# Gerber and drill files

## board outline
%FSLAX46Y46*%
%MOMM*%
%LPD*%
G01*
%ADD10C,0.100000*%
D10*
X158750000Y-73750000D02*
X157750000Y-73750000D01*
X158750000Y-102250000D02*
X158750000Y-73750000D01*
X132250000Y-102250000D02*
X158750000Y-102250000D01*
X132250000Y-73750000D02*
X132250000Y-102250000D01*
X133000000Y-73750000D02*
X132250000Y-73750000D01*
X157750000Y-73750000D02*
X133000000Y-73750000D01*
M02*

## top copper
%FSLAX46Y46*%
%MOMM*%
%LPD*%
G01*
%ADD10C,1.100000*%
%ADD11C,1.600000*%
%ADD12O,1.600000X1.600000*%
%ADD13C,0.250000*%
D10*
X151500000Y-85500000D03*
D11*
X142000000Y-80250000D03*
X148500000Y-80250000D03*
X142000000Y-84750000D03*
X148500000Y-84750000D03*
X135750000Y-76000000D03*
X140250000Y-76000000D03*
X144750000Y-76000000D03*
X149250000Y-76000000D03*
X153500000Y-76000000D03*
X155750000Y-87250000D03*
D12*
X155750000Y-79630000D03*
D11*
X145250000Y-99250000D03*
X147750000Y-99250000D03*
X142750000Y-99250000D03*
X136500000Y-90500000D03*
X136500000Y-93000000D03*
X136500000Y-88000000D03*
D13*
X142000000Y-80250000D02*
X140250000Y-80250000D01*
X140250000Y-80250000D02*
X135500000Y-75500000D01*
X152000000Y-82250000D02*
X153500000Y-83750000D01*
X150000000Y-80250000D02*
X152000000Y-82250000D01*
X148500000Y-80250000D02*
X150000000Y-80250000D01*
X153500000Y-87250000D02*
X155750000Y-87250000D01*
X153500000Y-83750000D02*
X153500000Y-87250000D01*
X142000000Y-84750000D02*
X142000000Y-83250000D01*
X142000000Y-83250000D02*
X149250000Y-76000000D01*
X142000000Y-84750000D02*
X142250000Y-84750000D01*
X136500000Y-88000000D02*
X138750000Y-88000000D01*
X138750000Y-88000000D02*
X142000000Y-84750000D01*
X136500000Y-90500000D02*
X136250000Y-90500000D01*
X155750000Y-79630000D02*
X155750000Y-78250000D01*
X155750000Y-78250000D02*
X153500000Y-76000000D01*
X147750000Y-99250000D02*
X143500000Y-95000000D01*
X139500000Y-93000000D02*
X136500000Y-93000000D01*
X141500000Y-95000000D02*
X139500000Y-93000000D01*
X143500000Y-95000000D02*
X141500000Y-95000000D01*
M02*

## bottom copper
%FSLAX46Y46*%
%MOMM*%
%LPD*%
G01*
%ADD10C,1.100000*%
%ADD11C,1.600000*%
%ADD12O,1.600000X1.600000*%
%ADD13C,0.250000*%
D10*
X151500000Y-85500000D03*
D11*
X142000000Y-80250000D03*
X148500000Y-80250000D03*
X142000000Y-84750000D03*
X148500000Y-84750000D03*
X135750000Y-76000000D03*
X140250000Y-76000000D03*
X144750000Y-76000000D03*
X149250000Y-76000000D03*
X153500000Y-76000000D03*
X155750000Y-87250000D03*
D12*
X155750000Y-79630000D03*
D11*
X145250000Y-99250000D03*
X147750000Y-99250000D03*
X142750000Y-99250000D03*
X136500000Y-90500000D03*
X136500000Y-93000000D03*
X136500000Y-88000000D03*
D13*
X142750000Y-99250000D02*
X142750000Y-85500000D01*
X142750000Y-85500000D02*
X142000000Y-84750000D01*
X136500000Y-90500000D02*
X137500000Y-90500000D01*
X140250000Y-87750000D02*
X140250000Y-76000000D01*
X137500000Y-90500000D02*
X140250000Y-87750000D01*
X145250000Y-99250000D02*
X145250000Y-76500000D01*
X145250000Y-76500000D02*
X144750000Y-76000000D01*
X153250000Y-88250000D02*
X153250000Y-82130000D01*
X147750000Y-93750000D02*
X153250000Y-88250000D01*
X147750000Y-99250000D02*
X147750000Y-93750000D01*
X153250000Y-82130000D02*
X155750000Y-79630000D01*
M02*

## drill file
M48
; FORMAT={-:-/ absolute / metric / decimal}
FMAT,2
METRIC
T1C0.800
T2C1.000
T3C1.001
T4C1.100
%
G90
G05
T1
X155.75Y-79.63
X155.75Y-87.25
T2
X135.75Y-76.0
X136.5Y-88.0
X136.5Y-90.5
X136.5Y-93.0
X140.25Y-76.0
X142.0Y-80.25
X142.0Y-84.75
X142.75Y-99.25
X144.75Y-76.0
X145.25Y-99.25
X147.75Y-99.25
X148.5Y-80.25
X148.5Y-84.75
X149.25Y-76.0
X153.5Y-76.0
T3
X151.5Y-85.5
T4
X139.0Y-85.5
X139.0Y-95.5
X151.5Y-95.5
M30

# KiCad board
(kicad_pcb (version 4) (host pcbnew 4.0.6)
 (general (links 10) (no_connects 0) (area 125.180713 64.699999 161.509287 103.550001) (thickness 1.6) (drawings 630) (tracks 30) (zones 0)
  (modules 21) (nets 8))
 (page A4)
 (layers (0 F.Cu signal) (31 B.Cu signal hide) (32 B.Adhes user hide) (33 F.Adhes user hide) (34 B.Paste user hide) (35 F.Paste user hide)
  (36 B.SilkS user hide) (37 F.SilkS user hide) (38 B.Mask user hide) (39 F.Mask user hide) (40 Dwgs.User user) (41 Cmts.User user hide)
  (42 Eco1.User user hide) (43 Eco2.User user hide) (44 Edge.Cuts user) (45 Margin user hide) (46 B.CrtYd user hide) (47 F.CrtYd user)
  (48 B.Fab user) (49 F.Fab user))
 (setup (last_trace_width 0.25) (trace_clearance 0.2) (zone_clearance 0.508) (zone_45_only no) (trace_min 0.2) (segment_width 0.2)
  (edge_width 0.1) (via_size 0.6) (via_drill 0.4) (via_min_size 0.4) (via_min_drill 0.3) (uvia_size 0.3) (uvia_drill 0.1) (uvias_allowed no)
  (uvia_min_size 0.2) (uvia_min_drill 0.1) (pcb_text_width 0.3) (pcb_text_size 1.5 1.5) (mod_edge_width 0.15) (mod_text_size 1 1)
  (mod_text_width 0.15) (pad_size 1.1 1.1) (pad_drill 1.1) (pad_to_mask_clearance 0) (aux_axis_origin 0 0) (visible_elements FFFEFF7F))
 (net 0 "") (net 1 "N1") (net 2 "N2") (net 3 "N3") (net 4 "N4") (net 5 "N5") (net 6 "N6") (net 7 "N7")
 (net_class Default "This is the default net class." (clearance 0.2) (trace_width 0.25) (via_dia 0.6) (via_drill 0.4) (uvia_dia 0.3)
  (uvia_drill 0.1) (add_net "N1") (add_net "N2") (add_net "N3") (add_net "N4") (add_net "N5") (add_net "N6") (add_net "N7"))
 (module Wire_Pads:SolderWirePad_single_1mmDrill (layer F.Cu) (at 151.5 95.5)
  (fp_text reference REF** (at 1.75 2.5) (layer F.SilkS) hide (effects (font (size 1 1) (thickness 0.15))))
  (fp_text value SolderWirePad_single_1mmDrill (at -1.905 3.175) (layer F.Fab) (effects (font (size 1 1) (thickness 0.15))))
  (pad "" np_thru_hole circle (at 0 0) (size 1.1 1.1) (drill 1.1) (layers *.Cu *.Mask)))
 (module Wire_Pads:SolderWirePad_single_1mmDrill (layer F.Cu) (at 139 95.5)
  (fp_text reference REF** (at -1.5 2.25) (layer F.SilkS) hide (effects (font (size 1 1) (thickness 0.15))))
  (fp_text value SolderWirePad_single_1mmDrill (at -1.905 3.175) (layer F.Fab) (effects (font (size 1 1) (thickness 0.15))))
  (pad "" np_thru_hole circle (at 0 0) (size 1.1 1.1) (drill 1.1) (layers *.Cu *.Mask)))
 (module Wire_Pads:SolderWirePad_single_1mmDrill (layer F.Cu) (at 151.5 85.5)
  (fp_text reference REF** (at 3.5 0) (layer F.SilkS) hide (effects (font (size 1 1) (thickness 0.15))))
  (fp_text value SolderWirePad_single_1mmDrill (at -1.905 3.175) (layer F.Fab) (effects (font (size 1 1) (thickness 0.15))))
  (pad "" np_thru_hole circle (at 0 0) (size 1.1 1.1) (drill 1.00076) (layers *.Cu *.Mask)))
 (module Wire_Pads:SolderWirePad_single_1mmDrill (layer F.Cu) (at 151.5 85.5)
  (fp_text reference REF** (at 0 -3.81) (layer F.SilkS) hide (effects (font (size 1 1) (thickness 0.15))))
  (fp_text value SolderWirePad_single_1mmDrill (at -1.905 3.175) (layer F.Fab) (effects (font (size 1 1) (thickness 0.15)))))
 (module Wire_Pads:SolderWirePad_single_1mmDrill (layer F.Cu) (at 142 80.25)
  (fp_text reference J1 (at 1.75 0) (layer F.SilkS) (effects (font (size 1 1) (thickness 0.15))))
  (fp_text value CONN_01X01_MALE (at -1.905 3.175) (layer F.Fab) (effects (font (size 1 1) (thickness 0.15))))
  (pad 1 thru_hole circle (at 0 0) (size 1.6 1.6) (drill 1) (layers *.Cu *.Mask) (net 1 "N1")))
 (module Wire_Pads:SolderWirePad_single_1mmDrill (layer F.Cu) (at 148.5 80.25)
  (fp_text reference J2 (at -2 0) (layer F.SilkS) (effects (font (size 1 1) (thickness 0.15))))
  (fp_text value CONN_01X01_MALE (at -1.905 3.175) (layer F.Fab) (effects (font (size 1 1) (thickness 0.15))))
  (pad 1 thru_hole circle (at 0 0) (size 1.6 1.6) (drill 1) (layers *.Cu *.Mask) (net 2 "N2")))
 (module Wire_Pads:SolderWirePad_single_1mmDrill (layer F.Cu) (at 142 84.75)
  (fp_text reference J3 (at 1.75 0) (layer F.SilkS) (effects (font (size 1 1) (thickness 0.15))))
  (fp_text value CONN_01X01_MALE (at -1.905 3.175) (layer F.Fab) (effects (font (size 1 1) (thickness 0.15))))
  (pad 1 thru_hole circle (at 0 0) (size 1.6 1.6) (drill 1) (layers *.Cu *.Mask) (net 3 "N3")))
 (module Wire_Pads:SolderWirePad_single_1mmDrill (layer F.Cu) (at 148.5 84.75)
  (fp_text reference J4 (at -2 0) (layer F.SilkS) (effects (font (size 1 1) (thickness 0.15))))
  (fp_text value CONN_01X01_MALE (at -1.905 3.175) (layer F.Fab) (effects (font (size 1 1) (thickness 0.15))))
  (pad 1 thru_hole circle (at 0 0) (size 1.6 1.6) (drill 1) (layers *.Cu *.Mask) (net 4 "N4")))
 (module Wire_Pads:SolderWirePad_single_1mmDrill (layer F.Cu) (at 135.5 71.25)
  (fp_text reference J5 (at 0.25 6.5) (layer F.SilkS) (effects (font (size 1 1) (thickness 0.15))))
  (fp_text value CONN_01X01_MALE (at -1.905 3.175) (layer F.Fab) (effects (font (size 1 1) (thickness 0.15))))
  (pad 1 thru_hole circle (at 0.25 4.75) (size 1.6 1.6) (drill 1) (layers *.Cu *.Mask) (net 1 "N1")))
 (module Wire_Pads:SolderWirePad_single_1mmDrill (layer F.Cu) (at 140 71.25)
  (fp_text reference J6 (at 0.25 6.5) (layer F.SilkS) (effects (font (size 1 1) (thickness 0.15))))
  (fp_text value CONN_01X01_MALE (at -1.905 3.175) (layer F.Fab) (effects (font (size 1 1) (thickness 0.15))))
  (pad 1 thru_hole circle (at 0.25 4.75) (size 1.6 1.6) (drill 1) (layers *.Cu *.Mask) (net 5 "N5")))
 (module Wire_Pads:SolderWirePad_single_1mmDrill (layer F.Cu) (at 144.5 71.25)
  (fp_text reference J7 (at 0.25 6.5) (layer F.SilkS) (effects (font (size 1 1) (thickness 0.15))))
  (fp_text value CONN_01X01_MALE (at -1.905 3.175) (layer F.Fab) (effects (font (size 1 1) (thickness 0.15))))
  (pad 1 thru_hole circle (at 0.25 4.75) (size 1.6 1.6) (drill 1) (layers *.Cu *.Mask) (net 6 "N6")))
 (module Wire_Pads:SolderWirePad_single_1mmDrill (layer F.Cu) (at 149 71.25)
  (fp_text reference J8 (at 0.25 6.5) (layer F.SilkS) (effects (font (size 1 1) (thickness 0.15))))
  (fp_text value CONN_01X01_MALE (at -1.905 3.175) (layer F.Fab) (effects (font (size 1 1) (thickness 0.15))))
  (pad 1 thru_hole circle (at 0.25 4.75) (size 1.6 1.6) (drill 1) (layers *.Cu *.Mask) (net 3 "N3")))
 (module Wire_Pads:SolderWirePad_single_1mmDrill (layer F.Cu) (at 153.5 71.25)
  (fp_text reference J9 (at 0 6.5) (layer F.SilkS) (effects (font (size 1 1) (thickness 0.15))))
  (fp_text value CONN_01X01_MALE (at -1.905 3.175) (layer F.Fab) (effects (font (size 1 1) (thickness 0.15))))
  (pad 1 thru_hole circle (at 0 4.75) (size 1.6 1.6) (drill 1) (layers *.Cu *.Mask) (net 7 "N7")))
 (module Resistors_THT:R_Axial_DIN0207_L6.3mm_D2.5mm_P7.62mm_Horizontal (layer F.Cu) (at 155.75 87.25 90)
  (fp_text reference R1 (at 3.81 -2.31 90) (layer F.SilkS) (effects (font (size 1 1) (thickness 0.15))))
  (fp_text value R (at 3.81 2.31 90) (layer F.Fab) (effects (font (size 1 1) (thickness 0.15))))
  (pad 1 thru_hole circle (at 0 0 90) (size 1.6 1.6) (drill 0.8) (layers *.Cu *.Mask) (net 2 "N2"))
  (pad 2 thru_hole oval (at 7.62 0 90) (size 1.6 1.6) (drill 0.8) (layers *.Cu *.Mask) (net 7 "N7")))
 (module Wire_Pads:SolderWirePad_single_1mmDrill (layer F.Cu) (at 145.25 99.25)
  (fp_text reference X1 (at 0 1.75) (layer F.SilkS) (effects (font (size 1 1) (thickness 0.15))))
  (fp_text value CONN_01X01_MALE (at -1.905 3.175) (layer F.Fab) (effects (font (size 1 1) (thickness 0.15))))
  (pad 1 thru_hole circle (at 0 0) (size 1.6 1.6) (drill 1) (layers *.Cu *.Mask) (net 6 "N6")))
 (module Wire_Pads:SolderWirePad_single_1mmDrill (layer F.Cu) (at 147.75 99.25)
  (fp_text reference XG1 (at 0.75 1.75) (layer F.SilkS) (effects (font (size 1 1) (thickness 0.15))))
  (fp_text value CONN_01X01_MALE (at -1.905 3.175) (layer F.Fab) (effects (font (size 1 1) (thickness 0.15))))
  (pad 1 thru_hole circle (at 0 0) (size 1.6 1.6) (drill 1) (layers *.Cu *.Mask) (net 7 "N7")))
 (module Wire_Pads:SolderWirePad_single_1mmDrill (layer F.Cu) (at 142.75 99.25)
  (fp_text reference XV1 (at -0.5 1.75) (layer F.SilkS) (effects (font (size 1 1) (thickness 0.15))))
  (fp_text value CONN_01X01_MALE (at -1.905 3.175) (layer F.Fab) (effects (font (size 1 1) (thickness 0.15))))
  (pad 1 thru_hole circle (at 0 0) (size 1.6 1.6) (drill 1) (layers *.Cu *.Mask) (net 3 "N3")))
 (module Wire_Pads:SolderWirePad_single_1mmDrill (layer F.Cu) (at 136.5 90.5)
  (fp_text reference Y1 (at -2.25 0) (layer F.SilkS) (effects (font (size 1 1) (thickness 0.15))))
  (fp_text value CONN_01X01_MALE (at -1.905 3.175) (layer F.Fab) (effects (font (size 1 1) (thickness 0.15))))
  (pad 1 thru_hole circle (at 0 0) (size 1.6 1.6) (drill 1) (layers *.Cu *.Mask) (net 5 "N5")))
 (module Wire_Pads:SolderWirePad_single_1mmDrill (layer F.Cu) (at 136.5 93)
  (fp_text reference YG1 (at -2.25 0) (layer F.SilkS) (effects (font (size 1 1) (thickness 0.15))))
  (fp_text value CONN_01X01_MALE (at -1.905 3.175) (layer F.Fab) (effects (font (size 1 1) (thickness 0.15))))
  (pad 1 thru_hole circle (at 0 0) (size 1.6 1.6) (drill 1) (layers *.Cu *.Mask) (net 7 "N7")))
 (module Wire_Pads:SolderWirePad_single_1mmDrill (layer F.Cu) (at 136.5 88)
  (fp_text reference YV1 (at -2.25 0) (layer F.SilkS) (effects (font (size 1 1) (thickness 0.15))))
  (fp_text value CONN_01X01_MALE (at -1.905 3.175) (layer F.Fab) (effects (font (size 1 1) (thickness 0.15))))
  (pad 1 thru_hole circle (at 0 0) (size 1.6 1.6) (drill 1) (layers *.Cu *.Mask) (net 3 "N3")))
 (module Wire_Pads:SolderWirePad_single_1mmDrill (layer F.Cu) (at 139 85.5)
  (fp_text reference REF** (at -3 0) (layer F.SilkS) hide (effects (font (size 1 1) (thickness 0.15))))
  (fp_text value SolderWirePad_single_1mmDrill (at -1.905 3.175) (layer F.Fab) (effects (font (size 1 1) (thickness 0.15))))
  (pad "" np_thru_hole circle (at 0 0) (size 1.1 1.1) (drill 1.1) (layers *.Cu *.Mask)))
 (gr_line (start 158.75 73.75) (end 157.75 73.75) (angle 90) (layer Edge.Cuts) (width 0.1))
 (gr_line (start 158.75 102.25) (end 158.75 73.75) (angle 90) (layer Edge.Cuts) (width 0.1))
 (gr_line (start 132.25 102.25) (end 158.75 102.25) (angle 90) (layer Edge.Cuts) (width 0.1))
 (gr_line (start 132.25 73.75) (end 132.25 102.25) (angle 90) (layer Edge.Cuts) (width 0.1))
 (gr_line (start 133 73.75) (end 132.25 73.75) (angle 90) (layer Edge.Cuts) (width 0.1))
 (gr_line (start 157.75 73.75) (end 133 73.75) (angle 90) (layer Edge.Cuts) (width 0.1))
 (segment (start 142 80.25) (end 140.25 80.25) (width 0.25) (layer F.Cu) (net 1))
 (segment (start 140.25 80.25) (end 135.5 75.5) (width 0.25) (layer F.Cu) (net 1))
 (segment (start 152 82.25) (end 153.5 83.75) (width 0.25) (layer F.Cu) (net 2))
 (segment (start 150 80.25) (end 152 82.25) (width 0.25) (layer F.Cu) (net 2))
 (segment (start 148.5 80.25) (end 150 80.25) (width 0.25) (layer F.Cu) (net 2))
 (segment (start 153.5 87.25) (end 155.75 87.25) (width 0.25) (layer F.Cu) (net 2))
 (segment (start 153.5 83.75) (end 153.5 87.25) (width 0.25) (layer F.Cu) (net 2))
 (segment (start 142 84.75) (end 142 83.25) (width 0.25) (layer F.Cu) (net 3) (status 400000))
 (segment (start 142 83.25) (end 149.25 76) (width 0.25) (layer F.Cu) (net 3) (status 800000))
 (segment (start 142.75 99.25) (end 142.75 85.5) (width 0.25) (layer B.Cu) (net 3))
 (segment (start 142.75 85.5) (end 142 84.75) (width 0.25) (layer B.Cu) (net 3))
 (segment (start 142 84.75) (end 142.25 84.75) (width 0.25) (layer F.Cu) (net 3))
 (segment (start 136.5 88) (end 138.75 88) (width 0.25) (layer F.Cu) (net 3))
 (segment (start 138.75 88) (end 142 84.75) (width 0.25) (layer F.Cu) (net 3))
 (segment (start 136.5 90.5) (end 137.5 90.5) (width 0.25) (layer B.Cu) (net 5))
 (segment (start 140.25 87.75) (end 140.25 76) (width 0.25) (layer B.Cu) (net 5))
 (segment (start 137.5 90.5) (end 140.25 87.75) (width 0.25) (layer B.Cu) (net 5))
 (segment (start 136.5 90.5) (end 136.25 90.5) (width 0.25) (layer F.Cu) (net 5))
 (segment (start 145.25 99.25) (end 145.25 76.5) (width 0.25) (layer B.Cu) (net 6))
 (segment (start 145.25 76.5) (end 144.75 76) (width 0.25) (layer B.Cu) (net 6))
 (segment (start 155.75 79.63) (end 155.75 78.25) (width 0.25) (layer F.Cu) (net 7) (status 400000))
 (segment (start 155.75 78.25) (end 153.5 76) (width 0.25) (layer F.Cu) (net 7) (status 800000))
 (segment (start 153.25 88.25) (end 153.25 82.13) (width 0.25) (layer B.Cu) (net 7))
 (segment (start 147.75 93.75) (end 153.25 88.25) (width 0.25) (layer B.Cu) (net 7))
 (segment (start 147.75 99.25) (end 147.75 93.75) (width 0.25) (layer B.Cu) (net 7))
 (segment (start 153.25 82.13) (end 155.75 79.63) (width 0.25) (layer B.Cu) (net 7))
 (segment (start 147.75 99.25) (end 143.5 95) (width 0.25) (layer F.Cu) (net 7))
 (segment (start 139.5 93) (end 136.5 93) (width 0.25) (layer F.Cu) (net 7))
 (segment (start 141.5 95) (end 139.5 93) (width 0.25) (layer F.Cu) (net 7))
 (segment (start 143.5 95) (end 141.5 95) (width 0.25) (layer F.Cu) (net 7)))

